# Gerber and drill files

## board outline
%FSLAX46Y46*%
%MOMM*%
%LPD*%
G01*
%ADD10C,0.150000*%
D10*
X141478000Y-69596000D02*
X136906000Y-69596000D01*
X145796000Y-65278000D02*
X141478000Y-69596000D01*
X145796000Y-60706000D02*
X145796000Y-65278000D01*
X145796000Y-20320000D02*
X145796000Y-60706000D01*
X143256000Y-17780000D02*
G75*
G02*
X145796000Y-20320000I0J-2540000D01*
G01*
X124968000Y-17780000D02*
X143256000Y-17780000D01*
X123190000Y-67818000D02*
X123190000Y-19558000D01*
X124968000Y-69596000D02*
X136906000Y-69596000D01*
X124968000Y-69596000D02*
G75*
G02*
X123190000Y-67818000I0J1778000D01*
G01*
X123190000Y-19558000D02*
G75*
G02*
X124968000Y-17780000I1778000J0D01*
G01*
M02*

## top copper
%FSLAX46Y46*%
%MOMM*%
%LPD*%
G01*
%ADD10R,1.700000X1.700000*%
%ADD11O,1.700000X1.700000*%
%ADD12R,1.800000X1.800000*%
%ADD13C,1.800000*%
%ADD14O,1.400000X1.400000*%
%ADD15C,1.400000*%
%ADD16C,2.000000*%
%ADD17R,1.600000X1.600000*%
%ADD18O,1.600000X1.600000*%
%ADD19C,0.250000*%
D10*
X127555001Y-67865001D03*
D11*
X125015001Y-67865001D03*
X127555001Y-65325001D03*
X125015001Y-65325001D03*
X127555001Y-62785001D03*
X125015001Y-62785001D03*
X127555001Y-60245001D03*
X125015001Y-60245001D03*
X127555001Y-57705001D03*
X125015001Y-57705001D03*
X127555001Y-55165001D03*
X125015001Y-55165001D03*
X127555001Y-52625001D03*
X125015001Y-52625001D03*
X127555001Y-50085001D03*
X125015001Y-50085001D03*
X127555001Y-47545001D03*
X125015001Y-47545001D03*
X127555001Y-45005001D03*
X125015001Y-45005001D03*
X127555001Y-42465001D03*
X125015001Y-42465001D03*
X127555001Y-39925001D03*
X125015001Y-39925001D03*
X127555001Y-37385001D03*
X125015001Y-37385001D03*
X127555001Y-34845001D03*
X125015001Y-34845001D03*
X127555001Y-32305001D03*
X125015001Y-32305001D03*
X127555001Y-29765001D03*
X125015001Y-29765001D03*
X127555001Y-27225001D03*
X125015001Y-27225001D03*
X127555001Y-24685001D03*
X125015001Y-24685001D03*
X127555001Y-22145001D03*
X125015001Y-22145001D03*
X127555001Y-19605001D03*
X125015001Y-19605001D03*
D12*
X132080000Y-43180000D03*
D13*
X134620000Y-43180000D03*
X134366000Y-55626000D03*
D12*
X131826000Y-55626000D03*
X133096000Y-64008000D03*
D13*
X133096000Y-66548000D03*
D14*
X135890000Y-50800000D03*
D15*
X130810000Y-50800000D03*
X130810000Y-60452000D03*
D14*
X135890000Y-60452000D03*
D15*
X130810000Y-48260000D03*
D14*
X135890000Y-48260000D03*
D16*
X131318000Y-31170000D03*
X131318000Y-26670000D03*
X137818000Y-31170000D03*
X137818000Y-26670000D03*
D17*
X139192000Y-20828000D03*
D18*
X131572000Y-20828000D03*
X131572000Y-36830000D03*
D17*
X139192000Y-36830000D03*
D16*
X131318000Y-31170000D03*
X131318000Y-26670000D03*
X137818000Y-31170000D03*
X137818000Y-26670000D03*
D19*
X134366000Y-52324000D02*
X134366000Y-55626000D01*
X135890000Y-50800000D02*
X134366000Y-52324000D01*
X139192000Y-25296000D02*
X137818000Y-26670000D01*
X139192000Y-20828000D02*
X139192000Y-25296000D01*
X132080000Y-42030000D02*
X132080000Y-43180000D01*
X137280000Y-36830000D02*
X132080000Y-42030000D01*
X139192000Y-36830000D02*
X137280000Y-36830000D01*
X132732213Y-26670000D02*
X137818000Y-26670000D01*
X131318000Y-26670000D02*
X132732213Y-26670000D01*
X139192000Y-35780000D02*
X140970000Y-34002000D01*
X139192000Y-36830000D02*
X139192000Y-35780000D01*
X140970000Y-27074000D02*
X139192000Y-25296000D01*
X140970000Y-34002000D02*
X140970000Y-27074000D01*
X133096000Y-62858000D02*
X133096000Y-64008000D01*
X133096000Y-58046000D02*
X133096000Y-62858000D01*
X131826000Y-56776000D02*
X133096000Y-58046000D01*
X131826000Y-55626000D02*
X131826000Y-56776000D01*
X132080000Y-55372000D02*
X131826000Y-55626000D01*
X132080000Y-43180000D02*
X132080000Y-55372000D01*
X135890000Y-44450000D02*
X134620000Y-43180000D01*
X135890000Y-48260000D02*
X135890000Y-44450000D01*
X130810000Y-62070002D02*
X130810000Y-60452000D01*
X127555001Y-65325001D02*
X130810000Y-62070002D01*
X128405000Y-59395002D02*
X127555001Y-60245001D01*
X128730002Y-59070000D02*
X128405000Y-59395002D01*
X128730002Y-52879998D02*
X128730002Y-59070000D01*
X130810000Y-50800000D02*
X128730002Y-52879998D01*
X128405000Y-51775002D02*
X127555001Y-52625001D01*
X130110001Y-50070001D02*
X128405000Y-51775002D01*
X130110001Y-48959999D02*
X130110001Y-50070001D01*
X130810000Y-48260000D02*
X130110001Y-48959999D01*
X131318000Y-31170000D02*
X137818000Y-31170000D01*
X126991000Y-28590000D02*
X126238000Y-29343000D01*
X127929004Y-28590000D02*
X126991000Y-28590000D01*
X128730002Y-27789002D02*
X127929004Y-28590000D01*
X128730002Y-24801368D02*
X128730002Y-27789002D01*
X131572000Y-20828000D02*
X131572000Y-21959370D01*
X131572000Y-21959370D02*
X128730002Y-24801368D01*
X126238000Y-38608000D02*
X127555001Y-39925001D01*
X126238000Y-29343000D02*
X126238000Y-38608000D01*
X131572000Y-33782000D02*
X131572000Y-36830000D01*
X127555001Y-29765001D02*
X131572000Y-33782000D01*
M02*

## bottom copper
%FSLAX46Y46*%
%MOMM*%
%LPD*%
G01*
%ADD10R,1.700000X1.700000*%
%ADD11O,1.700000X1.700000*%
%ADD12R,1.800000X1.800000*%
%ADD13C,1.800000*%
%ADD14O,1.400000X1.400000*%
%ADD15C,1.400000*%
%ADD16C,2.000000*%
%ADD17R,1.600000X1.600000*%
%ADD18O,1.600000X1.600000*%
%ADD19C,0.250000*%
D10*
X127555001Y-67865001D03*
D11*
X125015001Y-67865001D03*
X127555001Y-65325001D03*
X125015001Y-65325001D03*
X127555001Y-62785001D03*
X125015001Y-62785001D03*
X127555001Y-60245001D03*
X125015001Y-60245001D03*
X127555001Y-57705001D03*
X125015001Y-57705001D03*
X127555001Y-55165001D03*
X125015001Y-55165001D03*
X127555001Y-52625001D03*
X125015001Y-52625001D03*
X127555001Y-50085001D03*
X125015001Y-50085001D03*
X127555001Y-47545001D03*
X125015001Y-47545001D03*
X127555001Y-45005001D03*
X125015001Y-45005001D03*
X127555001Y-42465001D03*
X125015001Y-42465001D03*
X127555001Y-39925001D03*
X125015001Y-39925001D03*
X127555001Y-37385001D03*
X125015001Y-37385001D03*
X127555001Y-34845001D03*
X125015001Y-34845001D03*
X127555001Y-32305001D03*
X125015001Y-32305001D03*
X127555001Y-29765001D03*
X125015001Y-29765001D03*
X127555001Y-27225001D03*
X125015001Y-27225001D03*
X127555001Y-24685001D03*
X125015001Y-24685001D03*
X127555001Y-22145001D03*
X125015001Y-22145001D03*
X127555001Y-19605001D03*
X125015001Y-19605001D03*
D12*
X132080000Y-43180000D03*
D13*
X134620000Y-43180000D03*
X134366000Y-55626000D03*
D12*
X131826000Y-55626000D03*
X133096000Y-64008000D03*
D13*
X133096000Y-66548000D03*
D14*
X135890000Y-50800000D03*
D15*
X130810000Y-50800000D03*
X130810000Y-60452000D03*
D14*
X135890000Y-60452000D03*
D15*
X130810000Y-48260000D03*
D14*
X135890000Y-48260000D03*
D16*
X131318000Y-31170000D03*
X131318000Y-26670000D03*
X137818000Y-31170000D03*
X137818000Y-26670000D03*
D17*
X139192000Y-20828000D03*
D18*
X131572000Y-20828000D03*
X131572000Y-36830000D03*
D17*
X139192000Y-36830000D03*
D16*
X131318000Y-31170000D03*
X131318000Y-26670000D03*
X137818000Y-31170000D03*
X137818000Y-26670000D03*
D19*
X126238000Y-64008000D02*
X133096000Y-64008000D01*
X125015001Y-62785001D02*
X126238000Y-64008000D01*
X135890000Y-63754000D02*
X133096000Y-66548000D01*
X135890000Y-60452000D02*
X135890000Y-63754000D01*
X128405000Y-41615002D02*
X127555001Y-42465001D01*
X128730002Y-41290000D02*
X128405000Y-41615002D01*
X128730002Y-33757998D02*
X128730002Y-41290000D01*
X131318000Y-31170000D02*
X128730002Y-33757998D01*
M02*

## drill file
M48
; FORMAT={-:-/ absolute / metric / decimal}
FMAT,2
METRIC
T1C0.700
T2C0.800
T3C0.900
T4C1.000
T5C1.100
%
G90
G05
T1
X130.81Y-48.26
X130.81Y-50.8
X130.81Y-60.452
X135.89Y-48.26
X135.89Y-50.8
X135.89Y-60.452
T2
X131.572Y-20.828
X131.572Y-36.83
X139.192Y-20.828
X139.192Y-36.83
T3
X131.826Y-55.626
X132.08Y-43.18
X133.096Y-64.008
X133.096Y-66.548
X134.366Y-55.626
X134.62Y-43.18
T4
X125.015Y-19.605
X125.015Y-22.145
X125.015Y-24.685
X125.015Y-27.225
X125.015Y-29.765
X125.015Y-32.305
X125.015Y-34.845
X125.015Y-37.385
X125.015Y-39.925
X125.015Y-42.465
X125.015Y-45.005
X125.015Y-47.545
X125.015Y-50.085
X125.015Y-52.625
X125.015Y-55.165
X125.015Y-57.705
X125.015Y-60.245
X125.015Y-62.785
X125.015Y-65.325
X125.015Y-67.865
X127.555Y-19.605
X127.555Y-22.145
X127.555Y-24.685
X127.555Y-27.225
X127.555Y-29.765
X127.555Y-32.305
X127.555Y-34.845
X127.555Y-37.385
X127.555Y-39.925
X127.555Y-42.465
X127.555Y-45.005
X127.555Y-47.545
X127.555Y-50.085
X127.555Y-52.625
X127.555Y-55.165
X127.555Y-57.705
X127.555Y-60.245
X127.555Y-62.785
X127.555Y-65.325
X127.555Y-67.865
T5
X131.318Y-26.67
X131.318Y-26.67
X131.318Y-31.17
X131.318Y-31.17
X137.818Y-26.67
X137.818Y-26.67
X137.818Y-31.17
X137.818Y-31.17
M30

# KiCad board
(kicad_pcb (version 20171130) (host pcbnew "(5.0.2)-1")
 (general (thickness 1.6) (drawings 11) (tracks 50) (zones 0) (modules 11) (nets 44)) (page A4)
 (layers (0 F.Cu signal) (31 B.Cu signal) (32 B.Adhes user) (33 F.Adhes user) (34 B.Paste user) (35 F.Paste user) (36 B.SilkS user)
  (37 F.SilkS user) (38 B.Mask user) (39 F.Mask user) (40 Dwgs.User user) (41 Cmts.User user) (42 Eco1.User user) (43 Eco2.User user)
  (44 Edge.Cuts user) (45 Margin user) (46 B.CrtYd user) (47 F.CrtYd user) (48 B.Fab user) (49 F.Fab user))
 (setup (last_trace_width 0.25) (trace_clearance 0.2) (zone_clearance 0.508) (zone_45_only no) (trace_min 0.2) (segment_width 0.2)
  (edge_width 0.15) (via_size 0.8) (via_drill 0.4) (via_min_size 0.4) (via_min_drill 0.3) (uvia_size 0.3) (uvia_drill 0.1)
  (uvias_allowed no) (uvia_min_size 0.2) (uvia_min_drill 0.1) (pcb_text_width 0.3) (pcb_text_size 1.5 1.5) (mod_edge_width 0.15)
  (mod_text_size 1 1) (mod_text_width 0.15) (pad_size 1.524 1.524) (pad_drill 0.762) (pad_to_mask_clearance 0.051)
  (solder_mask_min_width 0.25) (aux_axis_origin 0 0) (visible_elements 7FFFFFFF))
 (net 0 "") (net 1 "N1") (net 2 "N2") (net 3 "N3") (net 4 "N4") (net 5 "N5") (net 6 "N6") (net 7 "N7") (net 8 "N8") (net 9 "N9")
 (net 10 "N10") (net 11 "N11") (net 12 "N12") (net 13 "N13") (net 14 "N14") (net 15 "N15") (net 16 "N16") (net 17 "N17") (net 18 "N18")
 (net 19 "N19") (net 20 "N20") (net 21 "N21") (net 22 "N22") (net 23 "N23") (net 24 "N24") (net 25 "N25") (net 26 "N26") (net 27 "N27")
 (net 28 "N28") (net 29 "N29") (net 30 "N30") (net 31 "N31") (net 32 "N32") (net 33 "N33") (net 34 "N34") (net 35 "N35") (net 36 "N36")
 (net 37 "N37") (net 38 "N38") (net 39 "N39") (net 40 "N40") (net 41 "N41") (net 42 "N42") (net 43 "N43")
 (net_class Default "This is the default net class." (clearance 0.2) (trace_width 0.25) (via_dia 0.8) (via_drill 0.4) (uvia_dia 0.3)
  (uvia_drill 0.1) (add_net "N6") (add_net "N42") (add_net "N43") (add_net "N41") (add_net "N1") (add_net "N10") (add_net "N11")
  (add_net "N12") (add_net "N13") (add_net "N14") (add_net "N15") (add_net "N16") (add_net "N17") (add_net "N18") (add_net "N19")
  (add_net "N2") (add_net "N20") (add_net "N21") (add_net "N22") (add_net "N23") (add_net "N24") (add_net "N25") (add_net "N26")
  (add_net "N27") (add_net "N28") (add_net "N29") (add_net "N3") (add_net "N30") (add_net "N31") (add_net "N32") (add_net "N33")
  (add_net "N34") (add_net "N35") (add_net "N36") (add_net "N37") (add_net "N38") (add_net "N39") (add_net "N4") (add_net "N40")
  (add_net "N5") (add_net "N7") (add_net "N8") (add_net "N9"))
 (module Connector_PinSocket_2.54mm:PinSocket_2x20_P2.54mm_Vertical (layer B.Cu) (at 127.555001 67.865001)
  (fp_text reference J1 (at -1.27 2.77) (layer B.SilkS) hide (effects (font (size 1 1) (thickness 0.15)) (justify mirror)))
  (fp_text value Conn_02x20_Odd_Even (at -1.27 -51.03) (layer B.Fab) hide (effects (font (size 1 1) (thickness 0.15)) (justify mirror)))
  (pad 1 thru_hole rect (at 0 0) (size 1.7 1.7) (drill 1) (layers *.Cu *.Mask) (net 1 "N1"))
  (pad 2 thru_hole oval (at -2.54 0) (size 1.7 1.7) (drill 1) (layers *.Cu *.Mask) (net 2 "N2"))
  (pad 3 thru_hole oval (at 0 -2.54) (size 1.7 1.7) (drill 1) (layers *.Cu *.Mask) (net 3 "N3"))
  (pad 4 thru_hole oval (at -2.54 -2.54) (size 1.7 1.7) (drill 1) (layers *.Cu *.Mask) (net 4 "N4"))
  (pad 5 thru_hole oval (at 0 -5.08) (size 1.7 1.7) (drill 1) (layers *.Cu *.Mask) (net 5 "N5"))
  (pad 6 thru_hole oval (at -2.54 -5.08) (size 1.7 1.7) (drill 1) (layers *.Cu *.Mask) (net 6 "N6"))
  (pad 7 thru_hole oval (at 0 -7.62) (size 1.7 1.7) (drill 1) (layers *.Cu *.Mask) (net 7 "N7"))
  (pad 8 thru_hole oval (at -2.54 -7.62) (size 1.7 1.7) (drill 1) (layers *.Cu *.Mask) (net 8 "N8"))
  (pad 9 thru_hole oval (at 0 -10.16) (size 1.7 1.7) (drill 1) (layers *.Cu *.Mask) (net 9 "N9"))
  (pad 10 thru_hole oval (at -2.54 -10.16) (size 1.7 1.7) (drill 1) (layers *.Cu *.Mask) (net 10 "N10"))
  (pad 11 thru_hole oval (at 0 -12.7) (size 1.7 1.7) (drill 1) (layers *.Cu *.Mask) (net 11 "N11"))
  (pad 12 thru_hole oval (at -2.54 -12.7) (size 1.7 1.7) (drill 1) (layers *.Cu *.Mask) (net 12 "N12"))
  (pad 13 thru_hole oval (at 0 -15.24) (size 1.7 1.7) (drill 1) (layers *.Cu *.Mask) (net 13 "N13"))
  (pad 14 thru_hole oval (at -2.54 -15.24) (size 1.7 1.7) (drill 1) (layers *.Cu *.Mask) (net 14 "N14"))
  (pad 15 thru_hole oval (at 0 -17.78) (size 1.7 1.7) (drill 1) (layers *.Cu *.Mask) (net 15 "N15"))
  (pad 16 thru_hole oval (at -2.54 -17.78) (size 1.7 1.7) (drill 1) (layers *.Cu *.Mask) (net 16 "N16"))
  (pad 17 thru_hole oval (at 0 -20.32) (size 1.7 1.7) (drill 1) (layers *.Cu *.Mask) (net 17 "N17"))
  (pad 18 thru_hole oval (at -2.54 -20.32) (size 1.7 1.7) (drill 1) (layers *.Cu *.Mask) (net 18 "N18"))
  (pad 19 thru_hole oval (at 0 -22.86) (size 1.7 1.7) (drill 1) (layers *.Cu *.Mask) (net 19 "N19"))
  (pad 20 thru_hole oval (at -2.54 -22.86) (size 1.7 1.7) (drill 1) (layers *.Cu *.Mask) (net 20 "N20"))
  (pad 21 thru_hole oval (at 0 -25.4) (size 1.7 1.7) (drill 1) (layers *.Cu *.Mask) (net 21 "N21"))
  (pad 22 thru_hole oval (at -2.54 -25.4) (size 1.7 1.7) (drill 1) (layers *.Cu *.Mask) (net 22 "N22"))
  (pad 23 thru_hole oval (at 0 -27.94) (size 1.7 1.7) (drill 1) (layers *.Cu *.Mask) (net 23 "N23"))
  (pad 24 thru_hole oval (at -2.54 -27.94) (size 1.7 1.7) (drill 1) (layers *.Cu *.Mask) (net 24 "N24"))
  (pad 25 thru_hole oval (at 0 -30.48) (size 1.7 1.7) (drill 1) (layers *.Cu *.Mask) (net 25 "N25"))
  (pad 26 thru_hole oval (at -2.54 -30.48) (size 1.7 1.7) (drill 1) (layers *.Cu *.Mask) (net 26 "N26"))
  (pad 27 thru_hole oval (at 0 -33.02) (size 1.7 1.7) (drill 1) (layers *.Cu *.Mask) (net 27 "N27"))
  (pad 28 thru_hole oval (at -2.54 -33.02) (size 1.7 1.7) (drill 1) (layers *.Cu *.Mask) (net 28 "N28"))
  (pad 29 thru_hole oval (at 0 -35.56) (size 1.7 1.7) (drill 1) (layers *.Cu *.Mask) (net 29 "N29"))
  (pad 30 thru_hole oval (at -2.54 -35.56) (size 1.7 1.7) (drill 1) (layers *.Cu *.Mask) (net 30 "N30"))
  (pad 31 thru_hole oval (at 0 -38.1) (size 1.7 1.7) (drill 1) (layers *.Cu *.Mask) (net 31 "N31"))
  (pad 32 thru_hole oval (at -2.54 -38.1) (size 1.7 1.7) (drill 1) (layers *.Cu *.Mask) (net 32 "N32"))
  (pad 33 thru_hole oval (at 0 -40.64) (size 1.7 1.7) (drill 1) (layers *.Cu *.Mask) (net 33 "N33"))
  (pad 34 thru_hole oval (at -2.54 -40.64) (size 1.7 1.7) (drill 1) (layers *.Cu *.Mask) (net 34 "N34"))
  (pad 35 thru_hole oval (at 0 -43.18) (size 1.7 1.7) (drill 1) (layers *.Cu *.Mask) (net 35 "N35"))
  (pad 36 thru_hole oval (at -2.54 -43.18) (size 1.7 1.7) (drill 1) (layers *.Cu *.Mask) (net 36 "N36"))
  (pad 37 thru_hole oval (at 0 -45.72) (size 1.7 1.7) (drill 1) (layers *.Cu *.Mask) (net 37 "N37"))
  (pad 38 thru_hole oval (at -2.54 -45.72) (size 1.7 1.7) (drill 1) (layers *.Cu *.Mask) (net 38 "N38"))
  (pad 39 thru_hole oval (at 0 -48.26) (size 1.7 1.7) (drill 1) (layers *.Cu *.Mask) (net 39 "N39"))
  (pad 40 thru_hole oval (at -2.54 -48.26) (size 1.7 1.7) (drill 1) (layers *.Cu *.Mask) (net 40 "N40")))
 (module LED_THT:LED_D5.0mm (layer F.Cu) (at 132.08 43.18)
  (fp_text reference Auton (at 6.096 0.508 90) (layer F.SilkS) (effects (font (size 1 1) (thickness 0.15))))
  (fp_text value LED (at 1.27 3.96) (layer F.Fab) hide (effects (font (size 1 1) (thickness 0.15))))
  (pad 1 thru_hole rect (at 0 0) (size 1.8 1.8) (drill 0.9) (layers *.Cu *.Mask) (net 6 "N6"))
  (pad 2 thru_hole circle (at 2.54 0) (size 1.8 1.8) (drill 0.9) (layers *.Cu *.Mask) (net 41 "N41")))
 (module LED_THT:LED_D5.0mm (layer F.Cu) (at 131.826 55.626)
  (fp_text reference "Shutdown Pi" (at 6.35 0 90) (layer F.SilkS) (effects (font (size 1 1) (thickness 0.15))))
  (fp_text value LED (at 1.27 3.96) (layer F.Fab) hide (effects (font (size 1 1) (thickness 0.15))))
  (pad 2 thru_hole circle (at 2.54 0) (size 1.8 1.8) (drill 0.9) (layers *.Cu *.Mask) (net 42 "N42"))
  (pad 1 thru_hole rect (at 0 0) (size 1.8 1.8) (drill 0.9) (layers *.Cu *.Mask) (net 6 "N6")))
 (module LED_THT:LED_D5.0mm (layer F.Cu) (at 133.096 64.008 270)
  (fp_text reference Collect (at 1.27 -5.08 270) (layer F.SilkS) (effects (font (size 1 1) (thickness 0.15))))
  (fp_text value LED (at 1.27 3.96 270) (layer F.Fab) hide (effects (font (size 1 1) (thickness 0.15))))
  (pad 1 thru_hole rect (at 0 0 270) (size 1.8 1.8) (drill 0.9) (layers *.Cu *.Mask) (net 6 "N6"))
  (pad 2 thru_hole circle (at 2.54 0 270) (size 1.8 1.8) (drill 0.9) (layers *.Cu *.Mask) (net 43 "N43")))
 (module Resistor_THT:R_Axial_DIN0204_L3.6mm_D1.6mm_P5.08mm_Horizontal (layer F.Cu) (at 130.81 50.8)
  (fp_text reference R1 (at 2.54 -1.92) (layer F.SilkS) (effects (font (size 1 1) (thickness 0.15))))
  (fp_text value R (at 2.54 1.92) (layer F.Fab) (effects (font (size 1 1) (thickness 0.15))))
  (pad 2 thru_hole oval (at 5.08 0) (size 1.4 1.4) (drill 0.7) (layers *.Cu *.Mask) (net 42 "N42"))
  (pad 1 thru_hole circle (at 0 0) (size 1.4 1.4) (drill 0.7) (layers *.Cu *.Mask) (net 7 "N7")))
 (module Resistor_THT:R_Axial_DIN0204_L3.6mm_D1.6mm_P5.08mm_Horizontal (layer F.Cu) (at 130.81 60.452)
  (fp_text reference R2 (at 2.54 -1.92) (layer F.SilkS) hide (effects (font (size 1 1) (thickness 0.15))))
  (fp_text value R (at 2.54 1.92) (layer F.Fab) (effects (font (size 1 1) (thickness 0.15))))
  (pad 1 thru_hole circle (at 0 0) (size 1.4 1.4) (drill 0.7) (layers *.Cu *.Mask) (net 3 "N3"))
  (pad 2 thru_hole oval (at 5.08 0) (size 1.4 1.4) (drill 0.7) (layers *.Cu *.Mask) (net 43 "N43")))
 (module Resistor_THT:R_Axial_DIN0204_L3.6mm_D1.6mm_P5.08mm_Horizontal (layer F.Cu) (at 130.81 48.26)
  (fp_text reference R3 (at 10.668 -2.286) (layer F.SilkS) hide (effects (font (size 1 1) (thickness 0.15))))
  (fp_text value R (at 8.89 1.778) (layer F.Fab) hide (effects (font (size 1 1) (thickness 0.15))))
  (pad 1 thru_hole circle (at 0 0) (size 1.4 1.4) (drill 0.7) (layers *.Cu *.Mask) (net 13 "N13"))
  (pad 2 thru_hole oval (at 5.08 0) (size 1.4 1.4) (drill 0.7) (layers *.Cu *.Mask) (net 41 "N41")))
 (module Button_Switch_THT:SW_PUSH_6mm (layer F.Cu) (at 131.318 26.67)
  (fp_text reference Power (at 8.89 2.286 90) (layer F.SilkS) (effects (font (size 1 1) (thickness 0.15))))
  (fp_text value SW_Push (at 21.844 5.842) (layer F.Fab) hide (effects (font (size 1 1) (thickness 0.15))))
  (pad 2 thru_hole circle (at 0 4.5 90) (size 2 2) (drill 1.1) (layers *.Cu *.Mask) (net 21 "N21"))
  (pad 1 thru_hole circle (at 0 0 90) (size 2 2) (drill 1.1) (layers *.Cu *.Mask) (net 6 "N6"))
  (pad 2 thru_hole circle (at 6.5 4.5 90) (size 2 2) (drill 1.1) (layers *.Cu *.Mask) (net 21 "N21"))
  (pad 1 thru_hole circle (at 6.5 0 90) (size 2 2) (drill 1.1) (layers *.Cu *.Mask) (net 6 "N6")))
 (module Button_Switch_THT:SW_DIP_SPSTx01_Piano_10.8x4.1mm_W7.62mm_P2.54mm (layer F.Cu) (at 139.192 20.828 180)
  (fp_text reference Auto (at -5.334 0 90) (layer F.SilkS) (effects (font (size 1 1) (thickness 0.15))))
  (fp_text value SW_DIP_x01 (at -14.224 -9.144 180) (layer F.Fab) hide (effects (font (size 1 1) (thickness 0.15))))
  (pad 1 thru_hole rect (at 0 0 180) (size 1.6 1.6) (drill 0.8) (layers *.Cu *.Mask) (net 6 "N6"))
  (pad 2 thru_hole oval (at 7.62 0 180) (size 1.6 1.6) (drill 0.8) (layers *.Cu *.Mask) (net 23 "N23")))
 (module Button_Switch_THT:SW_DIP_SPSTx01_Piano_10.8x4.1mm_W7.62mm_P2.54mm (layer F.Cu) (at 139.192 36.83 180)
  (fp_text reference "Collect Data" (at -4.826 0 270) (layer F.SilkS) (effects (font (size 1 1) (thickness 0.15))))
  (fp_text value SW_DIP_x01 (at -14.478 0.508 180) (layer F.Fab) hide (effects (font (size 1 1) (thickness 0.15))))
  (pad 2 thru_hole oval (at 7.62 0 180) (size 1.6 1.6) (drill 0.8) (layers *.Cu *.Mask) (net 31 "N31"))
  (pad 1 thru_hole rect (at 0 0 180) (size 1.6 1.6) (drill 0.8) (layers *.Cu *.Mask) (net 6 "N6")))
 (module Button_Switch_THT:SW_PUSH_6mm (layer F.Cu) (at 131.318 26.67)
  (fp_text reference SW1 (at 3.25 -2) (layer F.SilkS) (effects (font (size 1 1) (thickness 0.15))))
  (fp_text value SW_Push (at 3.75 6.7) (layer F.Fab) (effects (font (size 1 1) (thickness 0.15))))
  (pad 2 thru_hole circle (at 0 4.5 90) (size 2 2) (drill 1.1) (layers *.Cu *.Mask) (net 21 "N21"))
  (pad 1 thru_hole circle (at 0 0 90) (size 2 2) (drill 1.1) (layers *.Cu *.Mask) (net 6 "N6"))
  (pad 2 thru_hole circle (at 6.5 4.5 90) (size 2 2) (drill 1.1) (layers *.Cu *.Mask) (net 21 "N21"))
  (pad 1 thru_hole circle (at 6.5 0 90) (size 2 2) (drill 1.1) (layers *.Cu *.Mask) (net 6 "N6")))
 (gr_line (start 141.478 69.596) (end 136.906 69.596) (layer Edge.Cuts) (width 0.15))
 (gr_line (start 145.796 65.278) (end 141.478 69.596) (layer Edge.Cuts) (width 0.15))
 (gr_line (start 145.796 60.706) (end 145.796 65.278) (layer Edge.Cuts) (width 0.15))
 (gr_line (start 145.796 20.32) (end 145.796 60.706) (layer Edge.Cuts) (width 0.15))
 (gr_arc (start 143.256 20.32) (end 145.796 20.32) (angle -90) (layer Edge.Cuts) (width 0.15))
 (gr_line (start 124.968 17.78) (end 143.256 17.78) (layer Edge.Cuts) (width 0.15))
 (gr_line (start 123.19 67.818) (end 123.19 19.558) (layer Edge.Cuts) (width 0.15))
 (gr_line (start 124.968 69.596) (end 136.906 69.596) (layer Edge.Cuts) (width 0.15))
 (gr_arc (start 124.968 67.818) (end 123.19 67.818) (angle -90) (layer Edge.Cuts) (width 0.15))
 (gr_arc (start 124.968 19.558) (end 124.968 17.78) (angle -90) (layer Edge.Cuts) (width 0.15))
 (segment (start 134.366 52.324) (end 134.366 55.626) (width 0.25) (layer F.Cu) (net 42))
 (segment (start 135.89 50.8) (end 134.366 52.324) (width 0.25) (layer F.Cu) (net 42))
 (segment (start 139.192 25.296) (end 137.818 26.67) (width 0.25) (layer F.Cu) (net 6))
 (segment (start 139.192 20.828) (end 139.192 25.296) (width 0.25) (layer F.Cu) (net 6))
 (segment (start 132.08 42.03) (end 132.08 43.18) (width 0.25) (layer F.Cu) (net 6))
 (segment (start 137.28 36.83) (end 132.08 42.03) (width 0.25) (layer F.Cu) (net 6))
 (segment (start 139.192 36.83) (end 137.28 36.83) (width 0.25) (layer F.Cu) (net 6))
 (segment (start 132.732213 26.67) (end 137.818 26.67) (width 0.25) (layer F.Cu) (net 6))
 (segment (start 131.318 26.67) (end 132.732213 26.67) (width 0.25) (layer F.Cu) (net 6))
 (segment (start 139.192 35.78) (end 140.97 34.002) (width 0.25) (layer F.Cu) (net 6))
 (segment (start 139.192 36.83) (end 139.192 35.78) (width 0.25) (layer F.Cu) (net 6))
 (segment (start 140.97 27.074) (end 139.192 25.296) (width 0.25) (layer F.Cu) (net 6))
 (segment (start 140.97 34.002) (end 140.97 27.074) (width 0.25) (layer F.Cu) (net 6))
 (segment (start 126.238 64.008) (end 133.096 64.008) (width 0.25) (layer B.Cu) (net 6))
 (segment (start 125.015001 62.785001) (end 126.238 64.008) (width 0.25) (layer B.Cu) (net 6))
 (segment (start 133.096 62.858) (end 133.096 64.008) (width 0.25) (layer F.Cu) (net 6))
 (segment (start 133.096 58.046) (end 133.096 62.858) (width 0.25) (layer F.Cu) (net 6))
 (segment (start 131.826 56.776) (end 133.096 58.046) (width 0.25) (layer F.Cu) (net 6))
 (segment (start 131.826 55.626) (end 131.826 56.776) (width 0.25) (layer F.Cu) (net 6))
 (segment (start 132.08 55.372) (end 131.826 55.626) (width 0.25) (layer F.Cu) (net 6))
 (segment (start 132.08 43.18) (end 132.08 55.372) (width 0.25) (layer F.Cu) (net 6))
 (segment (start 135.89 63.754) (end 133.096 66.548) (width 0.25) (layer B.Cu) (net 43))
 (segment (start 135.89 60.452) (end 135.89 63.754) (width 0.25) (layer B.Cu) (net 43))
 (segment (start 135.89 44.45) (end 134.62 43.18) (width 0.25) (layer F.Cu) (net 41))
 (segment (start 135.89 48.26) (end 135.89 44.45) (width 0.25) (layer F.Cu) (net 41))
 (segment (start 130.81 62.070002) (end 130.81 60.452) (width 0.25) (layer F.Cu) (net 3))
 (segment (start 127.555001 65.325001) (end 130.81 62.070002) (width 0.25) (layer F.Cu) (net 3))
 (segment (start 128.405 59.395002) (end 127.555001 60.245001) (width 0.25) (layer F.Cu) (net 7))
 (segment (start 128.730002 59.07) (end 128.405 59.395002) (width 0.25) (layer F.Cu) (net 7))
 (segment (start 128.730002 52.879998) (end 128.730002 59.07) (width 0.25) (layer F.Cu) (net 7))
 (segment (start 130.81 50.8) (end 128.730002 52.879998) (width 0.25) (layer F.Cu) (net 7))
 (segment (start 128.405 51.775002) (end 127.555001 52.625001) (width 0.25) (layer F.Cu) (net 13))
 (segment (start 130.110001 50.070001) (end 128.405 51.775002) (width 0.25) (layer F.Cu) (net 13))
 (segment (start 130.110001 48.959999) (end 130.110001 50.070001) (width 0.25) (layer F.Cu) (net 13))
 (segment (start 130.81 48.26) (end 130.110001 48.959999) (width 0.25) (layer F.Cu) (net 13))
 (segment (start 131.318 31.17) (end 137.818 31.17) (width 0.25) (layer F.Cu) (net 21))
 (segment (start 128.405 41.615002) (end 127.555001 42.465001) (width 0.25) (layer B.Cu) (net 21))
 (segment (start 128.730002 41.29) (end 128.405 41.615002) (width 0.25) (layer B.Cu) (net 21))
 (segment (start 128.730002 33.757998) (end 128.730002 41.29) (width 0.25) (layer B.Cu) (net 21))
 (segment (start 131.318 31.17) (end 128.730002 33.757998) (width 0.25) (layer B.Cu) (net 21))
 (segment (start 126.991 28.59) (end 126.238 29.343) (width 0.25) (layer F.Cu) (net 23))
 (segment (start 127.929004 28.59) (end 126.991 28.59) (width 0.25) (layer F.Cu) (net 23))
 (segment (start 128.730002 27.789002) (end 127.929004 28.59) (width 0.25) (layer F.Cu) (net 23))
 (segment (start 128.730002 24.801368) (end 128.730002 27.789002) (width 0.25) (layer F.Cu) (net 23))
 (segment (start 131.572 20.828) (end 131.572 21.95937) (width 0.25) (layer F.Cu) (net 23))
 (segment (start 131.572 21.95937) (end 128.730002 24.801368) (width 0.25) (layer F.Cu) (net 23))
 (segment (start 126.238 38.608) (end 127.555001 39.925001) (width 0.25) (layer F.Cu) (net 23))
 (segment (start 126.238 29.343) (end 126.238 38.608) (width 0.25) (layer F.Cu) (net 23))
 (segment (start 131.572 33.782) (end 131.572 36.83) (width 0.25) (layer F.Cu) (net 31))
 (segment (start 127.555001 29.765001) (end 131.572 33.782) (width 0.25) (layer F.Cu) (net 31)))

